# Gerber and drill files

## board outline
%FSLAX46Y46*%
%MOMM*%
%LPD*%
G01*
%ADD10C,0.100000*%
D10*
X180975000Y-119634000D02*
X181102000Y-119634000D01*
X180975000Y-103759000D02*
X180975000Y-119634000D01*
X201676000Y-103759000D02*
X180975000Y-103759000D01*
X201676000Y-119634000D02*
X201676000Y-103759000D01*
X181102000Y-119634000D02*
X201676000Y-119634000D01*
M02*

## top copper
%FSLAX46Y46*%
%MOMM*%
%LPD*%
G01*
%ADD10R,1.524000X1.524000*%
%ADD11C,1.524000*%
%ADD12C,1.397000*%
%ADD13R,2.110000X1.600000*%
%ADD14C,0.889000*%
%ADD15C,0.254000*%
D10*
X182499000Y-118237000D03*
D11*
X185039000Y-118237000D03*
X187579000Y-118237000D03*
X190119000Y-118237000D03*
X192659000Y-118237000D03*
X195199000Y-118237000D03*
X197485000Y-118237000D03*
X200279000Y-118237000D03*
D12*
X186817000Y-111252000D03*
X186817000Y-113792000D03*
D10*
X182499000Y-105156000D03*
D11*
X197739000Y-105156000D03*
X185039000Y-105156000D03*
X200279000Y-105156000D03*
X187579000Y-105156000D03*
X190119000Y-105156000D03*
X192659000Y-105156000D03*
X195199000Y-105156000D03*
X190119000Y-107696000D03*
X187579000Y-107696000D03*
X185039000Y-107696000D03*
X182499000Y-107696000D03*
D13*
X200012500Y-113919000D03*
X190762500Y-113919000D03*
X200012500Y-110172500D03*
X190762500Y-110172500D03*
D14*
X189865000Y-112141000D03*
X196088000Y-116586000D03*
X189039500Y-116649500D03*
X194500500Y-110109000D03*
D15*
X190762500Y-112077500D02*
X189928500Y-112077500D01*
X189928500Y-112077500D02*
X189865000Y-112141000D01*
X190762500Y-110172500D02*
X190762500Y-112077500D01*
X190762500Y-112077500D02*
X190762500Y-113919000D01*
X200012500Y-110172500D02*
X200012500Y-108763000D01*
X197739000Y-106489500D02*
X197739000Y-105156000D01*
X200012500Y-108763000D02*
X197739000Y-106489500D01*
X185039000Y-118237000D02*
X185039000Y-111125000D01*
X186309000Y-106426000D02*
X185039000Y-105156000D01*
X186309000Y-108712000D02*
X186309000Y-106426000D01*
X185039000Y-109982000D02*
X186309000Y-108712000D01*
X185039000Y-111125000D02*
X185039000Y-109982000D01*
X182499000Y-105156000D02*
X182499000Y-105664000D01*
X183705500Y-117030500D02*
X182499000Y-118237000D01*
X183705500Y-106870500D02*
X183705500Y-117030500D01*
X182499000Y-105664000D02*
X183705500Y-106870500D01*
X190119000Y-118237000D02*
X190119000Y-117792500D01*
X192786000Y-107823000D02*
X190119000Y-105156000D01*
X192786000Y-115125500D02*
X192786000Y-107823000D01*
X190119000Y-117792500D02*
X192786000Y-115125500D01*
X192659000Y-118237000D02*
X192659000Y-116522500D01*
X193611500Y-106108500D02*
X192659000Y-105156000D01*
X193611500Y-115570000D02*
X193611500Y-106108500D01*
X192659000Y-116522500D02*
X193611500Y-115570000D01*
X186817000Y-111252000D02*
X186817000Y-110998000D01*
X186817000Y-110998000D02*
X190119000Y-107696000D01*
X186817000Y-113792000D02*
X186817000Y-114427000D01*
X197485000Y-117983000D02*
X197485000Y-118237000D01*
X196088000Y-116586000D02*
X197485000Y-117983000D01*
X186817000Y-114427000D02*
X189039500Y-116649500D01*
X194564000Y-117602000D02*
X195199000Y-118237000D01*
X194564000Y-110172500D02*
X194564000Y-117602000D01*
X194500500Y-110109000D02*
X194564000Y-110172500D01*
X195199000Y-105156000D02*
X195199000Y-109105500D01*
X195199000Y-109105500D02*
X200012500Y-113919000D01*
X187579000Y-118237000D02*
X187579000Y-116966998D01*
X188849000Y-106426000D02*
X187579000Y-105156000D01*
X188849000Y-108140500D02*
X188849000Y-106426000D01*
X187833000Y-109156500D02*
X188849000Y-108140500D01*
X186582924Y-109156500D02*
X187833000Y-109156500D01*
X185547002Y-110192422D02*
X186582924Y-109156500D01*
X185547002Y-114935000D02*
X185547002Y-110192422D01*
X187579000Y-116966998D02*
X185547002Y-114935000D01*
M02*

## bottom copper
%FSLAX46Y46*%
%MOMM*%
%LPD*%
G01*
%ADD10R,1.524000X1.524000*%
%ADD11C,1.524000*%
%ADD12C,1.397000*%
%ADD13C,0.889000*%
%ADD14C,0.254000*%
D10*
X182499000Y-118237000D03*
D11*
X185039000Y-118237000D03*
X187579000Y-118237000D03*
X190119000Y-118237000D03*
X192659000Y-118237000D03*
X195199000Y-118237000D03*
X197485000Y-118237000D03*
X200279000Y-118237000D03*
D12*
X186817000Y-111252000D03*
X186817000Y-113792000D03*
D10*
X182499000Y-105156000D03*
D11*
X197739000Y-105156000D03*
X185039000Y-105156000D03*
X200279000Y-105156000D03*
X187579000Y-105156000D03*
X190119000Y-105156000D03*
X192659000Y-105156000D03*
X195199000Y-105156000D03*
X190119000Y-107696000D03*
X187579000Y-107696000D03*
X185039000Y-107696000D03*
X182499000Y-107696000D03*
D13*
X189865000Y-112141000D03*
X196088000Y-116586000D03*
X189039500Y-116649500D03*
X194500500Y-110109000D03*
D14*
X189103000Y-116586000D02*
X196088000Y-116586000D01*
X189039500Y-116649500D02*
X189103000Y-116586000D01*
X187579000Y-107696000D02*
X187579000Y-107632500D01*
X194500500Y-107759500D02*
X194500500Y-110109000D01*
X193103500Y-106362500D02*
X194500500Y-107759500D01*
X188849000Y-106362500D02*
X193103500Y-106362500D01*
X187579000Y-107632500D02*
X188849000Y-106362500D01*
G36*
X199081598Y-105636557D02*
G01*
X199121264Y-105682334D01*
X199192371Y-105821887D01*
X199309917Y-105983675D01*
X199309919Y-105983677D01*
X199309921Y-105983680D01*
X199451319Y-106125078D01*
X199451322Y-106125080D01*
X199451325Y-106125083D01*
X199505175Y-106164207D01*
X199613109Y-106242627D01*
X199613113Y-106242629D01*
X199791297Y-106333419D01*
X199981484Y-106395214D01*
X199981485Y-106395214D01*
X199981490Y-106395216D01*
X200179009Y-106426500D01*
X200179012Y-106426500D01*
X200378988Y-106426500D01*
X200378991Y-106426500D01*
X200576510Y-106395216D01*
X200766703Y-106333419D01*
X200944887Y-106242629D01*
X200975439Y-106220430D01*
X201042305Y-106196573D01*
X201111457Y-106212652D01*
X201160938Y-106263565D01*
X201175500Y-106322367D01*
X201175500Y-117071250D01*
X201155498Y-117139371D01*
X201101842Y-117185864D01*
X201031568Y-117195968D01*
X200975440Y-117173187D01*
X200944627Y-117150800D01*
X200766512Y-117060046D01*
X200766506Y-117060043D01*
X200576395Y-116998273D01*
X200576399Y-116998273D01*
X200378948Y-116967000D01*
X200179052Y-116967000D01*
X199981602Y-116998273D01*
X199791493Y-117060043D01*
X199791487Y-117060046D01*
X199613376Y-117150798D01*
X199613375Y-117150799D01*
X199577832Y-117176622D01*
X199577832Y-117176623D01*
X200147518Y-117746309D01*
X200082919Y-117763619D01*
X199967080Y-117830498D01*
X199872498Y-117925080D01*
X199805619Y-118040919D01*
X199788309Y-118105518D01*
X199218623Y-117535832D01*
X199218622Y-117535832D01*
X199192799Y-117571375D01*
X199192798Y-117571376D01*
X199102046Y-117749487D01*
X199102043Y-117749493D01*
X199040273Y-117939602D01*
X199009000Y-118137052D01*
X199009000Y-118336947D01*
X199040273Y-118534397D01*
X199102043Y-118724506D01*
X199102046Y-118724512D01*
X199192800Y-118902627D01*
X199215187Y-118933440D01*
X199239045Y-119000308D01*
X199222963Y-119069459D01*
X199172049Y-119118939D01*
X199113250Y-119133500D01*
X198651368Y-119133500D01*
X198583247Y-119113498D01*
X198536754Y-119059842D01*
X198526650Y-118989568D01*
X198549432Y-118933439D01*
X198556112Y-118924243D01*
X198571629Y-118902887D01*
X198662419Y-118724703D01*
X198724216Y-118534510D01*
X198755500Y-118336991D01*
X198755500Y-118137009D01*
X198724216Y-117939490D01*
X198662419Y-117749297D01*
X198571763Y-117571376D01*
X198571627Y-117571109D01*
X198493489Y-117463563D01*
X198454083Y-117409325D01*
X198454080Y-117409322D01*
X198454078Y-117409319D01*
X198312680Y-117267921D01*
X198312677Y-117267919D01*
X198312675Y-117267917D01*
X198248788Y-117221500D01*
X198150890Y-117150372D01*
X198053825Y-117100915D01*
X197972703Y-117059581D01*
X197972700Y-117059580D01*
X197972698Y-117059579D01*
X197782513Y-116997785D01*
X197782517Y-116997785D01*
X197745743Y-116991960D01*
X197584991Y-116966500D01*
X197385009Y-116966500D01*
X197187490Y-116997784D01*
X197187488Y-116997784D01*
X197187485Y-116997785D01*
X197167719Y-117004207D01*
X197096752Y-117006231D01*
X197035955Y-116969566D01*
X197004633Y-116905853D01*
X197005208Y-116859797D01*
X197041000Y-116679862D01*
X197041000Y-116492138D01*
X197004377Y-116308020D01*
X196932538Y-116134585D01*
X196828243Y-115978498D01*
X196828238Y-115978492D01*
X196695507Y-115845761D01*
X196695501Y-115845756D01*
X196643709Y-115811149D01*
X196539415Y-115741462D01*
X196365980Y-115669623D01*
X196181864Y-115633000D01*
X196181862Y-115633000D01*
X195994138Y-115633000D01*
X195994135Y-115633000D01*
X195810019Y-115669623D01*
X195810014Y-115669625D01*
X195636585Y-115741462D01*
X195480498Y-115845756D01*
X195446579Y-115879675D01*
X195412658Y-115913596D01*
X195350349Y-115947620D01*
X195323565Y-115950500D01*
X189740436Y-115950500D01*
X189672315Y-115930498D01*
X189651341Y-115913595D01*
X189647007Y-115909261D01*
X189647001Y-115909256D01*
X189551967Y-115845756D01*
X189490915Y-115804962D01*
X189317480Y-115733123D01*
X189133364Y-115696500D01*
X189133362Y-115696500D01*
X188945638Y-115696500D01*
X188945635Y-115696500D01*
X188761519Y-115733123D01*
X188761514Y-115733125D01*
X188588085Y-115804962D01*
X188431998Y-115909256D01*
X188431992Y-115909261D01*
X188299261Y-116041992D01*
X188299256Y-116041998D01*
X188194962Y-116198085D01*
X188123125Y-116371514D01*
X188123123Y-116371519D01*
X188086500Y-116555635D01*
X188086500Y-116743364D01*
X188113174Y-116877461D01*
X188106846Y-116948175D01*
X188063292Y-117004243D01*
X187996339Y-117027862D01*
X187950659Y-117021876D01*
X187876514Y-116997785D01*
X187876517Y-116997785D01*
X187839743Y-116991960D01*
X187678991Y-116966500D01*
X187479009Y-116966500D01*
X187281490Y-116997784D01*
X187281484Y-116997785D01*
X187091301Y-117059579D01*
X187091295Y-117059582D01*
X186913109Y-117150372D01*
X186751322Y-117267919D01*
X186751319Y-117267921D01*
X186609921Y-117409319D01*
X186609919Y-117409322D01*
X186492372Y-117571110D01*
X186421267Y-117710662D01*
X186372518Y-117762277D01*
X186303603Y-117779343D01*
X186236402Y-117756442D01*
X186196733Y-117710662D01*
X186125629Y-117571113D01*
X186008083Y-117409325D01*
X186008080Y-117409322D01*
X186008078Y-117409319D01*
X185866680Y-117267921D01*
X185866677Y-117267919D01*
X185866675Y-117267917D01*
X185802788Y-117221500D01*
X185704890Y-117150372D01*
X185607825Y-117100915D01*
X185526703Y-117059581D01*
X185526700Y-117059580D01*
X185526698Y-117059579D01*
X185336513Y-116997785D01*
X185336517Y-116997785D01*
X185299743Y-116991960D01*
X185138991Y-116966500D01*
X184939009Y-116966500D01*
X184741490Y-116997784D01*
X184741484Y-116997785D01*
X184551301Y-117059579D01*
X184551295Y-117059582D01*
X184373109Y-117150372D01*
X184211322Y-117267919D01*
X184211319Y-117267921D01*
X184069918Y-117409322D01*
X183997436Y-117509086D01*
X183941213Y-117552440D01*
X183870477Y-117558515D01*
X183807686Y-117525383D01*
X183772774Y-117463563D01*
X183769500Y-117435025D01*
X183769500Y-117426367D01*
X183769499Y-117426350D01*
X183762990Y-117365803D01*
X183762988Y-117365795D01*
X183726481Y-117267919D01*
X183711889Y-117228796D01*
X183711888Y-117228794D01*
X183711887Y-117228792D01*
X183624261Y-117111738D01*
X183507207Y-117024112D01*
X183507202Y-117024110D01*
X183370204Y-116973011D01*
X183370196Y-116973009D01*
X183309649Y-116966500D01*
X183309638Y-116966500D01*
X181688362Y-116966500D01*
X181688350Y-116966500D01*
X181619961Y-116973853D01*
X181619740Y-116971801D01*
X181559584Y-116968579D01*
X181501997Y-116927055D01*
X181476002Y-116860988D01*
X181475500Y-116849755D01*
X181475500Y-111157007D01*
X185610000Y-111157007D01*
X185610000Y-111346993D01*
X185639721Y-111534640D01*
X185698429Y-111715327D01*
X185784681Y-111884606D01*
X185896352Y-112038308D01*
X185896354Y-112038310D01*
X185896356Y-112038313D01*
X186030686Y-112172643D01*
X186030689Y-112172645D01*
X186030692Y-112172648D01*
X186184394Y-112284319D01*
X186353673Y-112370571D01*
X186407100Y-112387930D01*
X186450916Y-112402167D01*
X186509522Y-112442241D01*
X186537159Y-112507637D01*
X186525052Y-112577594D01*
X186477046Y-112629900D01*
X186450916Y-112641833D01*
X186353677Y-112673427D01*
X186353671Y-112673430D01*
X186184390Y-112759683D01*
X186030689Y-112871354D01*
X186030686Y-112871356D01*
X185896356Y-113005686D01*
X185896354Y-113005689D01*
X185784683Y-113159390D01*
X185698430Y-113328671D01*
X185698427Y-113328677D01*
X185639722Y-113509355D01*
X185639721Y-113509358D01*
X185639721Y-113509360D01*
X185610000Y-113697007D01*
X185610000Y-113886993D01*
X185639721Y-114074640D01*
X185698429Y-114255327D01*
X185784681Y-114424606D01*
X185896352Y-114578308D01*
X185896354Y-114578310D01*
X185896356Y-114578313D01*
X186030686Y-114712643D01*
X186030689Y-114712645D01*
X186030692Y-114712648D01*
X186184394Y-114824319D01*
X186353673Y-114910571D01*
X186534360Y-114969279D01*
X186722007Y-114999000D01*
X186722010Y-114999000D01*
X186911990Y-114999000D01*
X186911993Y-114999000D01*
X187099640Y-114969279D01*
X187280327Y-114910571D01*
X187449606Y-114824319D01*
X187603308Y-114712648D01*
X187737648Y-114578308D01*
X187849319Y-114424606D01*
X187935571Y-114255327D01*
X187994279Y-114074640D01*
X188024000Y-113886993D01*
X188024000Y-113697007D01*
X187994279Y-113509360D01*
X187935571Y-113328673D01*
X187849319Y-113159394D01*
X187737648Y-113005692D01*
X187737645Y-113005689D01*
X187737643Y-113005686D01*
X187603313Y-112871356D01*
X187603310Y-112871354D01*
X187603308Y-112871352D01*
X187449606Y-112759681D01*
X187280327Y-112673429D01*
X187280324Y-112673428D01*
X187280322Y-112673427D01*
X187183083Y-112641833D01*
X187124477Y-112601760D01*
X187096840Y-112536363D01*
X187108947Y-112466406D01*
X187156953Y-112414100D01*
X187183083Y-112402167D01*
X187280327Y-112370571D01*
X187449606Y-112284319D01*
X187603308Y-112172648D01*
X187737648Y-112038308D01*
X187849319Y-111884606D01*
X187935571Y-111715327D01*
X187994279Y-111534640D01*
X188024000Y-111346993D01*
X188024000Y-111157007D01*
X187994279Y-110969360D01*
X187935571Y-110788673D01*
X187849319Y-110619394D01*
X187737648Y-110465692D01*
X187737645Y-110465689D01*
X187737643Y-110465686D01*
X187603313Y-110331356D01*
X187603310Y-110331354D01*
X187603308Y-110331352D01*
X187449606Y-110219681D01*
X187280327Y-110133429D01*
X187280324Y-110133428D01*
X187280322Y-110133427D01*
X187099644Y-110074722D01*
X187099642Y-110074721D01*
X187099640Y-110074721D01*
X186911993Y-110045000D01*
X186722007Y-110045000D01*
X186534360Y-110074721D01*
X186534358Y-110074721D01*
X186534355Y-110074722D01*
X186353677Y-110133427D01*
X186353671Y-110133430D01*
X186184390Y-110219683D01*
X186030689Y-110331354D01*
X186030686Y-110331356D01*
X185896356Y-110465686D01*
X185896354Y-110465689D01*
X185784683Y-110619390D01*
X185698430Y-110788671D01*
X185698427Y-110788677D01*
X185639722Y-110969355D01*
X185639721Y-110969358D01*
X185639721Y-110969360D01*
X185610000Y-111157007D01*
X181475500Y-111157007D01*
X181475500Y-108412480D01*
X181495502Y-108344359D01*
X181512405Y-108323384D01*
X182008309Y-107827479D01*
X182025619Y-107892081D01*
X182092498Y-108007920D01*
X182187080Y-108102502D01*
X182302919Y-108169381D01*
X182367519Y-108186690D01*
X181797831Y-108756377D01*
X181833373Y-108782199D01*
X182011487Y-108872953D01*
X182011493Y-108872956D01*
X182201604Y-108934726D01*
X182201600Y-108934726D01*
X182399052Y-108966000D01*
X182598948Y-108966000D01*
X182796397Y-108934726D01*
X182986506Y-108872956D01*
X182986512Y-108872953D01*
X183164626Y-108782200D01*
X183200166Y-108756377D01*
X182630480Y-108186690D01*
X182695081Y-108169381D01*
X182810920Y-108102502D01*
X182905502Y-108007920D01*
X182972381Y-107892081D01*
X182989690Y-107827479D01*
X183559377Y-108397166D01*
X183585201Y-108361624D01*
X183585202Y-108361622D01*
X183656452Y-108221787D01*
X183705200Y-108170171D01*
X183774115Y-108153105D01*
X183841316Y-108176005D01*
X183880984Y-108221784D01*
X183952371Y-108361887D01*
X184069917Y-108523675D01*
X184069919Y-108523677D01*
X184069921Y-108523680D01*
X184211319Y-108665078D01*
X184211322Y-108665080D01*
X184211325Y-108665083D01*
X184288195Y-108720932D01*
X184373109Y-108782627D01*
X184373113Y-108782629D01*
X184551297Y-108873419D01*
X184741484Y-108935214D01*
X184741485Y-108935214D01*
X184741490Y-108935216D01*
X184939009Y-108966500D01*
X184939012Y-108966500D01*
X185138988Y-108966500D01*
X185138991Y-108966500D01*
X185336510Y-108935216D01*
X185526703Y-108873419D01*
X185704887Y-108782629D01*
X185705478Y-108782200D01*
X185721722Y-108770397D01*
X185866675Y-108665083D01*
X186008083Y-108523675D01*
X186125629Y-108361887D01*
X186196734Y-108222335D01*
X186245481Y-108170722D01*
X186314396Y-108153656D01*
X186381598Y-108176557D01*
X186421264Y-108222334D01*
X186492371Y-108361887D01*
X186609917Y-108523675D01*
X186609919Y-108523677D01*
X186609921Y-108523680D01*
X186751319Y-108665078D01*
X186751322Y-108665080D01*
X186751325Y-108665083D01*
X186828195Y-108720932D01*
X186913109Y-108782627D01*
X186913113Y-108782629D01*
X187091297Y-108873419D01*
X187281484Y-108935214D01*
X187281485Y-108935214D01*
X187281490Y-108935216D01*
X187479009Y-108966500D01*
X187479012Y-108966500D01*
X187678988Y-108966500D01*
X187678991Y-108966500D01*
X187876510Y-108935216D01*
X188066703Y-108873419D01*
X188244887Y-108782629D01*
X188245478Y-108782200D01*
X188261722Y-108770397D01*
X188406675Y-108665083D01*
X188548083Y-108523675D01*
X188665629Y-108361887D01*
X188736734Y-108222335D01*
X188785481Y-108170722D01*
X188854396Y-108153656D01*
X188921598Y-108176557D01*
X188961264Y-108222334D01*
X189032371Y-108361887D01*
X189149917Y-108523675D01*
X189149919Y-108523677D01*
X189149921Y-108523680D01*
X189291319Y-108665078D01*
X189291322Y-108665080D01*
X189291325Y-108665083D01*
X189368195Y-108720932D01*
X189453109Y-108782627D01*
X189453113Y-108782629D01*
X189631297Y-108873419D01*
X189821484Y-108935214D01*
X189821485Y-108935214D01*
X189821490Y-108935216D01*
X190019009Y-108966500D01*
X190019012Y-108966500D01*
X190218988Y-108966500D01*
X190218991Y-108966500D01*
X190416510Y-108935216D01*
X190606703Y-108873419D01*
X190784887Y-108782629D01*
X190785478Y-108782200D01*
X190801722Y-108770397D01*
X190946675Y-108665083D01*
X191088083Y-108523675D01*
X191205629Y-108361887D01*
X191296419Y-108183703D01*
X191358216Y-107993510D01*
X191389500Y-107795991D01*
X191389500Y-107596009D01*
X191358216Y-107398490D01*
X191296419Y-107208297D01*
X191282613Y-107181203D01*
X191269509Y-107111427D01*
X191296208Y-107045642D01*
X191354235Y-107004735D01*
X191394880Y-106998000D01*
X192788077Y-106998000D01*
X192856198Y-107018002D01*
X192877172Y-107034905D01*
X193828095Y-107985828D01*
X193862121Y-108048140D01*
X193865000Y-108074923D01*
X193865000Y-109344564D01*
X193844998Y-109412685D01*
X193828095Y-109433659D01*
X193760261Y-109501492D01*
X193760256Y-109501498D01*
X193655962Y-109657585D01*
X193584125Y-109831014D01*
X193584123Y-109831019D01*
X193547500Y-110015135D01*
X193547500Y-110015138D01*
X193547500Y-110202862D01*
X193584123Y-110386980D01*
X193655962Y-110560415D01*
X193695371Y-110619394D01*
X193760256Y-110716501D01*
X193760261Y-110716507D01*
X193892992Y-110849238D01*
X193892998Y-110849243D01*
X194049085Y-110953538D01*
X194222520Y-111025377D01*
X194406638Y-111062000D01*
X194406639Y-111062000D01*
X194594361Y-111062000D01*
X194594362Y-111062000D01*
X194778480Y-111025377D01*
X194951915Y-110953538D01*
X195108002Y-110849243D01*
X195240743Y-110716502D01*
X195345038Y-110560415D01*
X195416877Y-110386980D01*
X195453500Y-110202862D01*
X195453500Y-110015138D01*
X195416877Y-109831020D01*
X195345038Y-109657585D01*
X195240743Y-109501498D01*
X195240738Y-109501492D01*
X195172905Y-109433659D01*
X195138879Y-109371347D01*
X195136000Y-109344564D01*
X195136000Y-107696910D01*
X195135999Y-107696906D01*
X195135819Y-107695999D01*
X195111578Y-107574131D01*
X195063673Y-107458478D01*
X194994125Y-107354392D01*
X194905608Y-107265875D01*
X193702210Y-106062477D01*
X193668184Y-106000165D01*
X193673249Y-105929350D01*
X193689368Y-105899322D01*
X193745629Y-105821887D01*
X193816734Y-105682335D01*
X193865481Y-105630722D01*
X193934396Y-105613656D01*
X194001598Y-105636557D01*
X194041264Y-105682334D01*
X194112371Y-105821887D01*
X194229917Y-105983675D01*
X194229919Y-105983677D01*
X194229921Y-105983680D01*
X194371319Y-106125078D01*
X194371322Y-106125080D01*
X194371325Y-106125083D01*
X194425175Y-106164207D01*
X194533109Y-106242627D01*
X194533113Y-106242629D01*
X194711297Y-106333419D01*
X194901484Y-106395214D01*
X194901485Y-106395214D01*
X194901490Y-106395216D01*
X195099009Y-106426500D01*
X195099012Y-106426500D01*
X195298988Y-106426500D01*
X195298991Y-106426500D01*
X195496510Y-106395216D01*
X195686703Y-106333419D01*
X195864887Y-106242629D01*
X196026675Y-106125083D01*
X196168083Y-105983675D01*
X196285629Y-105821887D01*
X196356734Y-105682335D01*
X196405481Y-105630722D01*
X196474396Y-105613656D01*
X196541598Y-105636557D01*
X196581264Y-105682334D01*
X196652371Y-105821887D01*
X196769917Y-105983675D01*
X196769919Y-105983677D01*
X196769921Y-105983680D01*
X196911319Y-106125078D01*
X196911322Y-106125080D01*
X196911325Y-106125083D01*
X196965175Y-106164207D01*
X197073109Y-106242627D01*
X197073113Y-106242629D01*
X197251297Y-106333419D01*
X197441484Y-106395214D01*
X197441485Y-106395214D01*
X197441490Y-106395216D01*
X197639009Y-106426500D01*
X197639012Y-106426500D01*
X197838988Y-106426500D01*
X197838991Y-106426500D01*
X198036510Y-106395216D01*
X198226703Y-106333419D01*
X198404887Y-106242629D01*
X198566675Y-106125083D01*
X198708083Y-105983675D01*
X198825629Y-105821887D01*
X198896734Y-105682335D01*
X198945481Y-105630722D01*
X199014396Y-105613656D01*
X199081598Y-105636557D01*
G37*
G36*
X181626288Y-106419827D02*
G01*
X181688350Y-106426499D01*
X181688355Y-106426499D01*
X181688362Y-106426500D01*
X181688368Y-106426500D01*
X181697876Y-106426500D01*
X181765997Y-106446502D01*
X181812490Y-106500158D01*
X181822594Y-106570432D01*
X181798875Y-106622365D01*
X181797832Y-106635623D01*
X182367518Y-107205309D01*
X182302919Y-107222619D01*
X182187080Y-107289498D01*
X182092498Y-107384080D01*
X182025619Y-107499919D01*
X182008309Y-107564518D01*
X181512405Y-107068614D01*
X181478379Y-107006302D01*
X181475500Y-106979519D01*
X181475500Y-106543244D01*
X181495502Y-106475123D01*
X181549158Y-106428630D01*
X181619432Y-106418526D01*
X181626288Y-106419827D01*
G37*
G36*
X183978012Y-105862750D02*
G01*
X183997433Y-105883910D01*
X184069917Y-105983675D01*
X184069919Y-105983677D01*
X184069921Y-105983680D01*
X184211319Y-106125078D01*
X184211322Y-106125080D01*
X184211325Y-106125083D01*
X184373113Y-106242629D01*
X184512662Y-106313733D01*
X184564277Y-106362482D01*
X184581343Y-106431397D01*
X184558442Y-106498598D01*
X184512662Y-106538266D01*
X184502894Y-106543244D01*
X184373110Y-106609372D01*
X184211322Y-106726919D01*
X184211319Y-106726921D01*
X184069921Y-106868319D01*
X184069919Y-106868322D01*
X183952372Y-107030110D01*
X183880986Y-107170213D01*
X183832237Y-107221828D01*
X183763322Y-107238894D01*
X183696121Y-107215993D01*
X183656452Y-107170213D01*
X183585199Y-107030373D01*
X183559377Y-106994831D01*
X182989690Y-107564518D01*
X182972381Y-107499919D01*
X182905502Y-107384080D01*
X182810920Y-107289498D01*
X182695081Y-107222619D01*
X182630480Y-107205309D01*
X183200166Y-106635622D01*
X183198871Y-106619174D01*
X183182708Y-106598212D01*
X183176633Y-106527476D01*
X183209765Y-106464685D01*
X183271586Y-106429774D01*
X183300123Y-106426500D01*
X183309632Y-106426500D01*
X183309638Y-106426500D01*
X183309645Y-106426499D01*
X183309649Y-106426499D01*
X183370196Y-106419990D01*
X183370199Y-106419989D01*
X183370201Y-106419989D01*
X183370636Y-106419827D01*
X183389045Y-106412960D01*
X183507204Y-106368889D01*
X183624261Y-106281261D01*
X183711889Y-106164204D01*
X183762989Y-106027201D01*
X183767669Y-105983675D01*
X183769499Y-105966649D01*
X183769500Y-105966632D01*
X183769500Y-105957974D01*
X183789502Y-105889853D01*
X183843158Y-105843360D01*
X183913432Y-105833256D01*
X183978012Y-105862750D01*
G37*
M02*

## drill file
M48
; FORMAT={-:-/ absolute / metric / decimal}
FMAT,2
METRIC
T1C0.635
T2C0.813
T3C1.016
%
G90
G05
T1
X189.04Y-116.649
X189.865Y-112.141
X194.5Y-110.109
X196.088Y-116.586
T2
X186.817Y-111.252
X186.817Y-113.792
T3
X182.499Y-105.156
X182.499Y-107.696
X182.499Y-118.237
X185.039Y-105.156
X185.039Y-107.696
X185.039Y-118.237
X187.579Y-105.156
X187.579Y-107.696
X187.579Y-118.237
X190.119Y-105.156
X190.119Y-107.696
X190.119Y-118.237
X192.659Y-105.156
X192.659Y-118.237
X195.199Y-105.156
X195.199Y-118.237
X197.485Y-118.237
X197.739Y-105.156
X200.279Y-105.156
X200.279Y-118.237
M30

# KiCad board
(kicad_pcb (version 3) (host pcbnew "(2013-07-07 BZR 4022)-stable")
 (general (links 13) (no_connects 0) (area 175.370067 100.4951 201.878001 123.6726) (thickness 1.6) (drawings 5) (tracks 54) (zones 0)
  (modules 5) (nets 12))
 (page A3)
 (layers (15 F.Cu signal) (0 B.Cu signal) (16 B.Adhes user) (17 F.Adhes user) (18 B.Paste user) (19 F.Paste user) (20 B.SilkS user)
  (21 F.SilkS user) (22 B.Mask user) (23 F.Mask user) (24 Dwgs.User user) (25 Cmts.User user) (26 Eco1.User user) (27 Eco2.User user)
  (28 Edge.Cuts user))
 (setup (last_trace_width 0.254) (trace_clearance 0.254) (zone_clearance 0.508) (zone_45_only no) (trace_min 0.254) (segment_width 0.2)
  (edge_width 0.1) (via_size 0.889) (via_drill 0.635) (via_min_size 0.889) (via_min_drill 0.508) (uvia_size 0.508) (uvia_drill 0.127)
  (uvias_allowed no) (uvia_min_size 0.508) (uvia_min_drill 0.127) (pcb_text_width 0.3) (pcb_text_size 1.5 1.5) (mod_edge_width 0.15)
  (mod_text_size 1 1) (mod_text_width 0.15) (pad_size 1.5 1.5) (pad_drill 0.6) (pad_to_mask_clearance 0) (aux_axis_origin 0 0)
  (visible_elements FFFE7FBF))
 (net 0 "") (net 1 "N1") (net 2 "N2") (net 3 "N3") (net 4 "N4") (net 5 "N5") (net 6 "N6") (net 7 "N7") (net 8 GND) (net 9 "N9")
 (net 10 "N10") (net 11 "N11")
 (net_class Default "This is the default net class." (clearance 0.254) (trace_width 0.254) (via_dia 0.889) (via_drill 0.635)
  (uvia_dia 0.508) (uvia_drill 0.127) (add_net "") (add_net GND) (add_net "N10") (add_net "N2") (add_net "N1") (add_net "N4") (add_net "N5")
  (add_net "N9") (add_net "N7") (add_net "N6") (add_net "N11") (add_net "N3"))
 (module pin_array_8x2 (layer F.Cu) (at 191.389 119.507)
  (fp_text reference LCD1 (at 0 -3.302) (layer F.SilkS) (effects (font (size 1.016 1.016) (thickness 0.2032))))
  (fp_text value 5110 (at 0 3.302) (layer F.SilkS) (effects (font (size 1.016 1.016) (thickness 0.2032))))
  (pad 1 thru_hole rect (at -8.89 -1.27) (size 1.524 1.524) (drill 1.016) (layers *.Cu *.Mask F.SilkS) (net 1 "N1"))
  (pad 2 thru_hole circle (at -6.35 -1.27) (size 1.524 1.524) (drill 1.016) (layers *.Cu *.Mask F.SilkS) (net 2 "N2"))
  (pad 3 thru_hole circle (at -3.81 -1.27) (size 1.524 1.524) (drill 1.016) (layers *.Cu *.Mask F.SilkS) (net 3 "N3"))
  (pad 4 thru_hole circle (at -1.27 -1.27) (size 1.524 1.524) (drill 1.016) (layers *.Cu *.Mask F.SilkS) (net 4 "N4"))
  (pad 5 thru_hole circle (at 1.27 -1.27) (size 1.524 1.524) (drill 1.016) (layers *.Cu *.Mask F.SilkS) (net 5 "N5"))
  (pad 6 thru_hole circle (at 3.81 -1.27) (size 1.524 1.524) (drill 1.016) (layers *.Cu *.Mask F.SilkS) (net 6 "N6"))
  (pad 7 thru_hole circle (at 6.096 -1.27) (size 1.524 1.524) (drill 1.016) (layers *.Cu *.Mask F.SilkS) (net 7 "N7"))
  (pad 8 thru_hole circle (at 8.89 -1.27) (size 1.524 1.524) (drill 1.016) (layers *.Cu *.Mask F.SilkS) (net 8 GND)))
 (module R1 (layer F.Cu) (at 186.817 112.522 270) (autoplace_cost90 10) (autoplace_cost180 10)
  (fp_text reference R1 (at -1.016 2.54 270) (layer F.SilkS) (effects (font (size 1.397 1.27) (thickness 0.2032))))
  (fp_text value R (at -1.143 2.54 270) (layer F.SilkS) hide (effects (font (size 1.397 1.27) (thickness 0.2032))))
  (pad 1 thru_hole circle (at -1.27 0 270) (size 1.397 1.397) (drill 0.8128) (layers *.Cu *.Mask F.SilkS) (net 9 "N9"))
  (pad 2 thru_hole circle (at 1.27 0 270) (size 1.397 1.397) (drill 0.8128) (layers *.Cu *.Mask F.SilkS) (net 7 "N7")))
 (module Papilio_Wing (layer F.Cu) (at 182.499 105.156)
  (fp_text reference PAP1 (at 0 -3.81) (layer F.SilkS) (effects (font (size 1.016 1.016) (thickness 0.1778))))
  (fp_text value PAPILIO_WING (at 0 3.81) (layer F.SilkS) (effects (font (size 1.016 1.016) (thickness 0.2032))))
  (pad 1 thru_hole rect (at 0 0) (size 1.524 1.524) (drill 1.016) (layers *.Cu *.Mask F.SilkS) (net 1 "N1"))
  (pad 7 thru_hole circle (at 15.24 0) (size 1.524 1.524) (drill 1.016) (layers *.Cu *.Mask F.SilkS) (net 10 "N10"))
  (pad 2 thru_hole circle (at 2.54 0) (size 1.524 1.524) (drill 1.016) (layers *.Cu *.Mask F.SilkS) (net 2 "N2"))
  (pad 8 thru_hole circle (at 17.78 0) (size 1.524 1.524) (drill 1.016) (layers *.Cu *.Mask F.SilkS))
  (pad 3 thru_hole circle (at 5.08 0) (size 1.524 1.524) (drill 1.016) (layers *.Cu *.Mask F.SilkS) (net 3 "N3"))
  (pad 4 thru_hole circle (at 7.62 0) (size 1.524 1.524) (drill 1.016) (layers *.Cu *.Mask F.SilkS) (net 4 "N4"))
  (pad 5 thru_hole circle (at 10.16 0) (size 1.524 1.524) (drill 1.016) (layers *.Cu *.Mask F.SilkS) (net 5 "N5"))
  (pad 6 thru_hole circle (at 12.7 0) (size 1.524 1.524) (drill 1.016) (layers *.Cu *.Mask F.SilkS) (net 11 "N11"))
  (pad 9 thru_hole circle (at 7.62 2.54) (size 1.524 1.524) (drill 1.016) (layers *.Cu *.Mask F.SilkS) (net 9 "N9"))
  (pad 10 thru_hole circle (at 5.08 2.54) (size 1.524 1.524) (drill 1.016) (layers *.Cu *.Mask F.SilkS) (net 6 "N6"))
  (pad 11 thru_hole circle (at 2.54 2.54) (size 1.524 1.524) (drill 1.016) (layers *.Cu *.Mask F.SilkS))
  (pad 12 thru_hole circle (at 0 2.54) (size 1.524 1.524) (drill 1.016) (layers *.Cu *.Mask F.SilkS) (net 8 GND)))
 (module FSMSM (layer F.Cu) (at 195.2625 113.919 180)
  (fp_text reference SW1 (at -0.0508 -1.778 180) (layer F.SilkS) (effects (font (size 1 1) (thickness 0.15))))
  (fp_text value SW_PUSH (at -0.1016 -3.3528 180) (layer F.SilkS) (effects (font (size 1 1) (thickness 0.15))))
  (pad 1 smd rect (at -4.75 0 180) (size 2.11 1.6) (layers F.Cu F.Paste F.Mask) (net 11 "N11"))
  (pad 2 smd rect (at 4.5 0 180) (size 2.11 1.6) (layers F.Cu F.Paste F.Mask) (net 8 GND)))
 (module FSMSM (layer F.Cu) (at 195.2625 110.1725 180)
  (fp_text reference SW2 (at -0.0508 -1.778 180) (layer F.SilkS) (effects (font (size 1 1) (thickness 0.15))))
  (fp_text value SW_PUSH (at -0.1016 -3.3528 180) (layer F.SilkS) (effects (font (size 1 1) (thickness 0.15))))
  (pad 1 smd rect (at -4.75 0 180) (size 2.11 1.6) (layers F.Cu F.Paste F.Mask) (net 10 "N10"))
  (pad 2 smd rect (at 4.5 0 180) (size 2.11 1.6) (layers F.Cu F.Paste F.Mask) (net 8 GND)))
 (gr_line (start 180.975 119.634) (end 181.102 119.634) (angle 90) (layer Edge.Cuts) (width 0.1))
 (gr_line (start 180.975 103.759) (end 180.975 119.634) (angle 90) (layer Edge.Cuts) (width 0.1))
 (gr_line (start 201.676 103.759) (end 180.975 103.759) (angle 90) (layer Edge.Cuts) (width 0.1))
 (gr_line (start 201.676 119.634) (end 201.676 103.759) (angle 90) (layer Edge.Cuts) (width 0.1))
 (gr_line (start 181.102 119.634) (end 201.676 119.634) (angle 90) (layer Edge.Cuts) (width 0.1))
 (segment (start 190.7625 112.0775) (end 189.9285 112.0775) (width 0.254) (layer F.Cu) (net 8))
 (via (at 189.865 112.141) (size 0.889) (layers F.Cu B.Cu) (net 8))
 (segment (start 189.9285 112.0775) (end 189.865 112.141) (width 0.254) (layer F.Cu) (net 8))
 (segment (start 190.7625 110.1725) (end 190.7625 112.0775) (width 0.254) (layer F.Cu) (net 8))
 (segment (start 190.7625 112.0775) (end 190.7625 113.919) (width 0.254) (layer F.Cu) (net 8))
 (segment (start 200.0125 110.1725) (end 200.0125 108.763) (width 0.254) (layer F.Cu) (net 10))
 (segment (start 197.739 106.4895) (end 197.739 105.156) (width 0.254) (layer F.Cu) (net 10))
 (segment (start 200.0125 108.763) (end 197.739 106.4895) (width 0.254) (layer F.Cu) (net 10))
 (segment (start 185.039 118.237) (end 185.039 111.125) (width 0.254) (layer F.Cu) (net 2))
 (segment (start 186.309 106.426) (end 185.039 105.156) (width 0.254) (layer F.Cu) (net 2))
 (segment (start 186.309 108.712) (end 186.309 106.426) (width 0.254) (layer F.Cu) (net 2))
 (segment (start 185.039 109.982) (end 186.309 108.712) (width 0.254) (layer F.Cu) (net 2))
 (segment (start 185.039 111.125) (end 185.039 109.982) (width 0.254) (layer F.Cu) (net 2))
 (segment (start 182.499 105.156) (end 182.499 105.664) (width 0.254) (layer F.Cu) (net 1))
 (segment (start 183.7055 117.0305) (end 182.499 118.237) (width 0.254) (layer F.Cu) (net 1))
 (segment (start 183.7055 106.8705) (end 183.7055 117.0305) (width 0.254) (layer F.Cu) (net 1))
 (segment (start 182.499 105.664) (end 183.7055 106.8705) (width 0.254) (layer F.Cu) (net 1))
 (segment (start 190.119 118.237) (end 190.119 117.7925) (width 0.254) (layer F.Cu) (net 4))
 (segment (start 192.786 107.823) (end 190.119 105.156) (width 0.254) (layer F.Cu) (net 4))
 (segment (start 192.786 115.1255) (end 192.786 107.823) (width 0.254) (layer F.Cu) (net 4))
 (segment (start 190.119 117.7925) (end 192.786 115.1255) (width 0.254) (layer F.Cu) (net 4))
 (segment (start 192.659 118.237) (end 192.659 116.5225) (width 0.254) (layer F.Cu) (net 5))
 (segment (start 193.6115 106.1085) (end 192.659 105.156) (width 0.254) (layer F.Cu) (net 5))
 (segment (start 193.6115 115.57) (end 193.6115 106.1085) (width 0.254) (layer F.Cu) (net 5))
 (segment (start 192.659 116.5225) (end 193.6115 115.57) (width 0.254) (layer F.Cu) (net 5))
 (segment (start 186.817 111.252) (end 186.817 110.998) (width 0.254) (layer F.Cu) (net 9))
 (segment (start 186.817 110.998) (end 190.119 107.696) (width 0.254) (layer F.Cu) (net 9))
 (segment (start 186.817 113.792) (end 186.817 114.427) (width 0.254) (layer F.Cu) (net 7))
 (segment (start 197.485 117.983) (end 197.485 118.237) (width 0.254) (layer F.Cu) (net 7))
 (segment (start 196.088 116.586) (end 197.485 117.983) (width 0.254) (layer F.Cu) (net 7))
 (via (at 196.088 116.586) (size 0.889) (layers F.Cu B.Cu) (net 7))
 (segment (start 189.103 116.586) (end 196.088 116.586) (width 0.254) (layer B.Cu) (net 7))
 (segment (start 189.0395 116.6495) (end 189.103 116.586) (width 0.254) (layer B.Cu) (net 7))
 (via (at 189.0395 116.6495) (size 0.889) (layers F.Cu B.Cu) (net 7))
 (segment (start 186.817 114.427) (end 189.0395 116.6495) (width 0.254) (layer F.Cu) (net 7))
 (segment (start 187.579 107.696) (end 187.579 107.6325) (width 0.254) (layer B.Cu) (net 6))
 (segment (start 194.564 117.602) (end 195.199 118.237) (width 0.254) (layer F.Cu) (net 6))
 (segment (start 194.564 110.1725) (end 194.564 117.602) (width 0.254) (layer F.Cu) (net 6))
 (segment (start 194.5005 110.109) (end 194.564 110.1725) (width 0.254) (layer F.Cu) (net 6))
 (via (at 194.5005 110.109) (size 0.889) (layers F.Cu B.Cu) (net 6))
 (segment (start 194.5005 107.7595) (end 194.5005 110.109) (width 0.254) (layer B.Cu) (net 6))
 (segment (start 193.1035 106.3625) (end 194.5005 107.7595) (width 0.254) (layer B.Cu) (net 6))
 (segment (start 188.849 106.3625) (end 193.1035 106.3625) (width 0.254) (layer B.Cu) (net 6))
 (segment (start 187.579 107.6325) (end 188.849 106.3625) (width 0.254) (layer B.Cu) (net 6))
 (segment (start 195.199 105.156) (end 195.199 109.1055) (width 0.254) (layer F.Cu) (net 11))
 (segment (start 195.199 109.1055) (end 200.0125 113.919) (width 0.254) (layer F.Cu) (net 11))
 (segment (start 187.579 118.237) (end 187.579 116.966998) (width 0.254) (layer F.Cu) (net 3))
 (segment (start 188.849 106.426) (end 187.579 105.156) (width 0.254) (layer F.Cu) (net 3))
 (segment (start 188.849 108.1405) (end 188.849 106.426) (width 0.254) (layer F.Cu) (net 3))
 (segment (start 187.833 109.1565) (end 188.849 108.1405) (width 0.254) (layer F.Cu) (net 3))
 (segment (start 186.582924 109.1565) (end 187.833 109.1565) (width 0.254) (layer F.Cu) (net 3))
 (segment (start 185.547002 110.192422) (end 186.582924 109.1565) (width 0.254) (layer F.Cu) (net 3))
 (segment (start 185.547002 114.935) (end 185.547002 110.192422) (width 0.254) (layer F.Cu) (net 3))
 (segment (start 187.579 116.966998) (end 185.547002 114.935) (width 0.254) (layer F.Cu) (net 3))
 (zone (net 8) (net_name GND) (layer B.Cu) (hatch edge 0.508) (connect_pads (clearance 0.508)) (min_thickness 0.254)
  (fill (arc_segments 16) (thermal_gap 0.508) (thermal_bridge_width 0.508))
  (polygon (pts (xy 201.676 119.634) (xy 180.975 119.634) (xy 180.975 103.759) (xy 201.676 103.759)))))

